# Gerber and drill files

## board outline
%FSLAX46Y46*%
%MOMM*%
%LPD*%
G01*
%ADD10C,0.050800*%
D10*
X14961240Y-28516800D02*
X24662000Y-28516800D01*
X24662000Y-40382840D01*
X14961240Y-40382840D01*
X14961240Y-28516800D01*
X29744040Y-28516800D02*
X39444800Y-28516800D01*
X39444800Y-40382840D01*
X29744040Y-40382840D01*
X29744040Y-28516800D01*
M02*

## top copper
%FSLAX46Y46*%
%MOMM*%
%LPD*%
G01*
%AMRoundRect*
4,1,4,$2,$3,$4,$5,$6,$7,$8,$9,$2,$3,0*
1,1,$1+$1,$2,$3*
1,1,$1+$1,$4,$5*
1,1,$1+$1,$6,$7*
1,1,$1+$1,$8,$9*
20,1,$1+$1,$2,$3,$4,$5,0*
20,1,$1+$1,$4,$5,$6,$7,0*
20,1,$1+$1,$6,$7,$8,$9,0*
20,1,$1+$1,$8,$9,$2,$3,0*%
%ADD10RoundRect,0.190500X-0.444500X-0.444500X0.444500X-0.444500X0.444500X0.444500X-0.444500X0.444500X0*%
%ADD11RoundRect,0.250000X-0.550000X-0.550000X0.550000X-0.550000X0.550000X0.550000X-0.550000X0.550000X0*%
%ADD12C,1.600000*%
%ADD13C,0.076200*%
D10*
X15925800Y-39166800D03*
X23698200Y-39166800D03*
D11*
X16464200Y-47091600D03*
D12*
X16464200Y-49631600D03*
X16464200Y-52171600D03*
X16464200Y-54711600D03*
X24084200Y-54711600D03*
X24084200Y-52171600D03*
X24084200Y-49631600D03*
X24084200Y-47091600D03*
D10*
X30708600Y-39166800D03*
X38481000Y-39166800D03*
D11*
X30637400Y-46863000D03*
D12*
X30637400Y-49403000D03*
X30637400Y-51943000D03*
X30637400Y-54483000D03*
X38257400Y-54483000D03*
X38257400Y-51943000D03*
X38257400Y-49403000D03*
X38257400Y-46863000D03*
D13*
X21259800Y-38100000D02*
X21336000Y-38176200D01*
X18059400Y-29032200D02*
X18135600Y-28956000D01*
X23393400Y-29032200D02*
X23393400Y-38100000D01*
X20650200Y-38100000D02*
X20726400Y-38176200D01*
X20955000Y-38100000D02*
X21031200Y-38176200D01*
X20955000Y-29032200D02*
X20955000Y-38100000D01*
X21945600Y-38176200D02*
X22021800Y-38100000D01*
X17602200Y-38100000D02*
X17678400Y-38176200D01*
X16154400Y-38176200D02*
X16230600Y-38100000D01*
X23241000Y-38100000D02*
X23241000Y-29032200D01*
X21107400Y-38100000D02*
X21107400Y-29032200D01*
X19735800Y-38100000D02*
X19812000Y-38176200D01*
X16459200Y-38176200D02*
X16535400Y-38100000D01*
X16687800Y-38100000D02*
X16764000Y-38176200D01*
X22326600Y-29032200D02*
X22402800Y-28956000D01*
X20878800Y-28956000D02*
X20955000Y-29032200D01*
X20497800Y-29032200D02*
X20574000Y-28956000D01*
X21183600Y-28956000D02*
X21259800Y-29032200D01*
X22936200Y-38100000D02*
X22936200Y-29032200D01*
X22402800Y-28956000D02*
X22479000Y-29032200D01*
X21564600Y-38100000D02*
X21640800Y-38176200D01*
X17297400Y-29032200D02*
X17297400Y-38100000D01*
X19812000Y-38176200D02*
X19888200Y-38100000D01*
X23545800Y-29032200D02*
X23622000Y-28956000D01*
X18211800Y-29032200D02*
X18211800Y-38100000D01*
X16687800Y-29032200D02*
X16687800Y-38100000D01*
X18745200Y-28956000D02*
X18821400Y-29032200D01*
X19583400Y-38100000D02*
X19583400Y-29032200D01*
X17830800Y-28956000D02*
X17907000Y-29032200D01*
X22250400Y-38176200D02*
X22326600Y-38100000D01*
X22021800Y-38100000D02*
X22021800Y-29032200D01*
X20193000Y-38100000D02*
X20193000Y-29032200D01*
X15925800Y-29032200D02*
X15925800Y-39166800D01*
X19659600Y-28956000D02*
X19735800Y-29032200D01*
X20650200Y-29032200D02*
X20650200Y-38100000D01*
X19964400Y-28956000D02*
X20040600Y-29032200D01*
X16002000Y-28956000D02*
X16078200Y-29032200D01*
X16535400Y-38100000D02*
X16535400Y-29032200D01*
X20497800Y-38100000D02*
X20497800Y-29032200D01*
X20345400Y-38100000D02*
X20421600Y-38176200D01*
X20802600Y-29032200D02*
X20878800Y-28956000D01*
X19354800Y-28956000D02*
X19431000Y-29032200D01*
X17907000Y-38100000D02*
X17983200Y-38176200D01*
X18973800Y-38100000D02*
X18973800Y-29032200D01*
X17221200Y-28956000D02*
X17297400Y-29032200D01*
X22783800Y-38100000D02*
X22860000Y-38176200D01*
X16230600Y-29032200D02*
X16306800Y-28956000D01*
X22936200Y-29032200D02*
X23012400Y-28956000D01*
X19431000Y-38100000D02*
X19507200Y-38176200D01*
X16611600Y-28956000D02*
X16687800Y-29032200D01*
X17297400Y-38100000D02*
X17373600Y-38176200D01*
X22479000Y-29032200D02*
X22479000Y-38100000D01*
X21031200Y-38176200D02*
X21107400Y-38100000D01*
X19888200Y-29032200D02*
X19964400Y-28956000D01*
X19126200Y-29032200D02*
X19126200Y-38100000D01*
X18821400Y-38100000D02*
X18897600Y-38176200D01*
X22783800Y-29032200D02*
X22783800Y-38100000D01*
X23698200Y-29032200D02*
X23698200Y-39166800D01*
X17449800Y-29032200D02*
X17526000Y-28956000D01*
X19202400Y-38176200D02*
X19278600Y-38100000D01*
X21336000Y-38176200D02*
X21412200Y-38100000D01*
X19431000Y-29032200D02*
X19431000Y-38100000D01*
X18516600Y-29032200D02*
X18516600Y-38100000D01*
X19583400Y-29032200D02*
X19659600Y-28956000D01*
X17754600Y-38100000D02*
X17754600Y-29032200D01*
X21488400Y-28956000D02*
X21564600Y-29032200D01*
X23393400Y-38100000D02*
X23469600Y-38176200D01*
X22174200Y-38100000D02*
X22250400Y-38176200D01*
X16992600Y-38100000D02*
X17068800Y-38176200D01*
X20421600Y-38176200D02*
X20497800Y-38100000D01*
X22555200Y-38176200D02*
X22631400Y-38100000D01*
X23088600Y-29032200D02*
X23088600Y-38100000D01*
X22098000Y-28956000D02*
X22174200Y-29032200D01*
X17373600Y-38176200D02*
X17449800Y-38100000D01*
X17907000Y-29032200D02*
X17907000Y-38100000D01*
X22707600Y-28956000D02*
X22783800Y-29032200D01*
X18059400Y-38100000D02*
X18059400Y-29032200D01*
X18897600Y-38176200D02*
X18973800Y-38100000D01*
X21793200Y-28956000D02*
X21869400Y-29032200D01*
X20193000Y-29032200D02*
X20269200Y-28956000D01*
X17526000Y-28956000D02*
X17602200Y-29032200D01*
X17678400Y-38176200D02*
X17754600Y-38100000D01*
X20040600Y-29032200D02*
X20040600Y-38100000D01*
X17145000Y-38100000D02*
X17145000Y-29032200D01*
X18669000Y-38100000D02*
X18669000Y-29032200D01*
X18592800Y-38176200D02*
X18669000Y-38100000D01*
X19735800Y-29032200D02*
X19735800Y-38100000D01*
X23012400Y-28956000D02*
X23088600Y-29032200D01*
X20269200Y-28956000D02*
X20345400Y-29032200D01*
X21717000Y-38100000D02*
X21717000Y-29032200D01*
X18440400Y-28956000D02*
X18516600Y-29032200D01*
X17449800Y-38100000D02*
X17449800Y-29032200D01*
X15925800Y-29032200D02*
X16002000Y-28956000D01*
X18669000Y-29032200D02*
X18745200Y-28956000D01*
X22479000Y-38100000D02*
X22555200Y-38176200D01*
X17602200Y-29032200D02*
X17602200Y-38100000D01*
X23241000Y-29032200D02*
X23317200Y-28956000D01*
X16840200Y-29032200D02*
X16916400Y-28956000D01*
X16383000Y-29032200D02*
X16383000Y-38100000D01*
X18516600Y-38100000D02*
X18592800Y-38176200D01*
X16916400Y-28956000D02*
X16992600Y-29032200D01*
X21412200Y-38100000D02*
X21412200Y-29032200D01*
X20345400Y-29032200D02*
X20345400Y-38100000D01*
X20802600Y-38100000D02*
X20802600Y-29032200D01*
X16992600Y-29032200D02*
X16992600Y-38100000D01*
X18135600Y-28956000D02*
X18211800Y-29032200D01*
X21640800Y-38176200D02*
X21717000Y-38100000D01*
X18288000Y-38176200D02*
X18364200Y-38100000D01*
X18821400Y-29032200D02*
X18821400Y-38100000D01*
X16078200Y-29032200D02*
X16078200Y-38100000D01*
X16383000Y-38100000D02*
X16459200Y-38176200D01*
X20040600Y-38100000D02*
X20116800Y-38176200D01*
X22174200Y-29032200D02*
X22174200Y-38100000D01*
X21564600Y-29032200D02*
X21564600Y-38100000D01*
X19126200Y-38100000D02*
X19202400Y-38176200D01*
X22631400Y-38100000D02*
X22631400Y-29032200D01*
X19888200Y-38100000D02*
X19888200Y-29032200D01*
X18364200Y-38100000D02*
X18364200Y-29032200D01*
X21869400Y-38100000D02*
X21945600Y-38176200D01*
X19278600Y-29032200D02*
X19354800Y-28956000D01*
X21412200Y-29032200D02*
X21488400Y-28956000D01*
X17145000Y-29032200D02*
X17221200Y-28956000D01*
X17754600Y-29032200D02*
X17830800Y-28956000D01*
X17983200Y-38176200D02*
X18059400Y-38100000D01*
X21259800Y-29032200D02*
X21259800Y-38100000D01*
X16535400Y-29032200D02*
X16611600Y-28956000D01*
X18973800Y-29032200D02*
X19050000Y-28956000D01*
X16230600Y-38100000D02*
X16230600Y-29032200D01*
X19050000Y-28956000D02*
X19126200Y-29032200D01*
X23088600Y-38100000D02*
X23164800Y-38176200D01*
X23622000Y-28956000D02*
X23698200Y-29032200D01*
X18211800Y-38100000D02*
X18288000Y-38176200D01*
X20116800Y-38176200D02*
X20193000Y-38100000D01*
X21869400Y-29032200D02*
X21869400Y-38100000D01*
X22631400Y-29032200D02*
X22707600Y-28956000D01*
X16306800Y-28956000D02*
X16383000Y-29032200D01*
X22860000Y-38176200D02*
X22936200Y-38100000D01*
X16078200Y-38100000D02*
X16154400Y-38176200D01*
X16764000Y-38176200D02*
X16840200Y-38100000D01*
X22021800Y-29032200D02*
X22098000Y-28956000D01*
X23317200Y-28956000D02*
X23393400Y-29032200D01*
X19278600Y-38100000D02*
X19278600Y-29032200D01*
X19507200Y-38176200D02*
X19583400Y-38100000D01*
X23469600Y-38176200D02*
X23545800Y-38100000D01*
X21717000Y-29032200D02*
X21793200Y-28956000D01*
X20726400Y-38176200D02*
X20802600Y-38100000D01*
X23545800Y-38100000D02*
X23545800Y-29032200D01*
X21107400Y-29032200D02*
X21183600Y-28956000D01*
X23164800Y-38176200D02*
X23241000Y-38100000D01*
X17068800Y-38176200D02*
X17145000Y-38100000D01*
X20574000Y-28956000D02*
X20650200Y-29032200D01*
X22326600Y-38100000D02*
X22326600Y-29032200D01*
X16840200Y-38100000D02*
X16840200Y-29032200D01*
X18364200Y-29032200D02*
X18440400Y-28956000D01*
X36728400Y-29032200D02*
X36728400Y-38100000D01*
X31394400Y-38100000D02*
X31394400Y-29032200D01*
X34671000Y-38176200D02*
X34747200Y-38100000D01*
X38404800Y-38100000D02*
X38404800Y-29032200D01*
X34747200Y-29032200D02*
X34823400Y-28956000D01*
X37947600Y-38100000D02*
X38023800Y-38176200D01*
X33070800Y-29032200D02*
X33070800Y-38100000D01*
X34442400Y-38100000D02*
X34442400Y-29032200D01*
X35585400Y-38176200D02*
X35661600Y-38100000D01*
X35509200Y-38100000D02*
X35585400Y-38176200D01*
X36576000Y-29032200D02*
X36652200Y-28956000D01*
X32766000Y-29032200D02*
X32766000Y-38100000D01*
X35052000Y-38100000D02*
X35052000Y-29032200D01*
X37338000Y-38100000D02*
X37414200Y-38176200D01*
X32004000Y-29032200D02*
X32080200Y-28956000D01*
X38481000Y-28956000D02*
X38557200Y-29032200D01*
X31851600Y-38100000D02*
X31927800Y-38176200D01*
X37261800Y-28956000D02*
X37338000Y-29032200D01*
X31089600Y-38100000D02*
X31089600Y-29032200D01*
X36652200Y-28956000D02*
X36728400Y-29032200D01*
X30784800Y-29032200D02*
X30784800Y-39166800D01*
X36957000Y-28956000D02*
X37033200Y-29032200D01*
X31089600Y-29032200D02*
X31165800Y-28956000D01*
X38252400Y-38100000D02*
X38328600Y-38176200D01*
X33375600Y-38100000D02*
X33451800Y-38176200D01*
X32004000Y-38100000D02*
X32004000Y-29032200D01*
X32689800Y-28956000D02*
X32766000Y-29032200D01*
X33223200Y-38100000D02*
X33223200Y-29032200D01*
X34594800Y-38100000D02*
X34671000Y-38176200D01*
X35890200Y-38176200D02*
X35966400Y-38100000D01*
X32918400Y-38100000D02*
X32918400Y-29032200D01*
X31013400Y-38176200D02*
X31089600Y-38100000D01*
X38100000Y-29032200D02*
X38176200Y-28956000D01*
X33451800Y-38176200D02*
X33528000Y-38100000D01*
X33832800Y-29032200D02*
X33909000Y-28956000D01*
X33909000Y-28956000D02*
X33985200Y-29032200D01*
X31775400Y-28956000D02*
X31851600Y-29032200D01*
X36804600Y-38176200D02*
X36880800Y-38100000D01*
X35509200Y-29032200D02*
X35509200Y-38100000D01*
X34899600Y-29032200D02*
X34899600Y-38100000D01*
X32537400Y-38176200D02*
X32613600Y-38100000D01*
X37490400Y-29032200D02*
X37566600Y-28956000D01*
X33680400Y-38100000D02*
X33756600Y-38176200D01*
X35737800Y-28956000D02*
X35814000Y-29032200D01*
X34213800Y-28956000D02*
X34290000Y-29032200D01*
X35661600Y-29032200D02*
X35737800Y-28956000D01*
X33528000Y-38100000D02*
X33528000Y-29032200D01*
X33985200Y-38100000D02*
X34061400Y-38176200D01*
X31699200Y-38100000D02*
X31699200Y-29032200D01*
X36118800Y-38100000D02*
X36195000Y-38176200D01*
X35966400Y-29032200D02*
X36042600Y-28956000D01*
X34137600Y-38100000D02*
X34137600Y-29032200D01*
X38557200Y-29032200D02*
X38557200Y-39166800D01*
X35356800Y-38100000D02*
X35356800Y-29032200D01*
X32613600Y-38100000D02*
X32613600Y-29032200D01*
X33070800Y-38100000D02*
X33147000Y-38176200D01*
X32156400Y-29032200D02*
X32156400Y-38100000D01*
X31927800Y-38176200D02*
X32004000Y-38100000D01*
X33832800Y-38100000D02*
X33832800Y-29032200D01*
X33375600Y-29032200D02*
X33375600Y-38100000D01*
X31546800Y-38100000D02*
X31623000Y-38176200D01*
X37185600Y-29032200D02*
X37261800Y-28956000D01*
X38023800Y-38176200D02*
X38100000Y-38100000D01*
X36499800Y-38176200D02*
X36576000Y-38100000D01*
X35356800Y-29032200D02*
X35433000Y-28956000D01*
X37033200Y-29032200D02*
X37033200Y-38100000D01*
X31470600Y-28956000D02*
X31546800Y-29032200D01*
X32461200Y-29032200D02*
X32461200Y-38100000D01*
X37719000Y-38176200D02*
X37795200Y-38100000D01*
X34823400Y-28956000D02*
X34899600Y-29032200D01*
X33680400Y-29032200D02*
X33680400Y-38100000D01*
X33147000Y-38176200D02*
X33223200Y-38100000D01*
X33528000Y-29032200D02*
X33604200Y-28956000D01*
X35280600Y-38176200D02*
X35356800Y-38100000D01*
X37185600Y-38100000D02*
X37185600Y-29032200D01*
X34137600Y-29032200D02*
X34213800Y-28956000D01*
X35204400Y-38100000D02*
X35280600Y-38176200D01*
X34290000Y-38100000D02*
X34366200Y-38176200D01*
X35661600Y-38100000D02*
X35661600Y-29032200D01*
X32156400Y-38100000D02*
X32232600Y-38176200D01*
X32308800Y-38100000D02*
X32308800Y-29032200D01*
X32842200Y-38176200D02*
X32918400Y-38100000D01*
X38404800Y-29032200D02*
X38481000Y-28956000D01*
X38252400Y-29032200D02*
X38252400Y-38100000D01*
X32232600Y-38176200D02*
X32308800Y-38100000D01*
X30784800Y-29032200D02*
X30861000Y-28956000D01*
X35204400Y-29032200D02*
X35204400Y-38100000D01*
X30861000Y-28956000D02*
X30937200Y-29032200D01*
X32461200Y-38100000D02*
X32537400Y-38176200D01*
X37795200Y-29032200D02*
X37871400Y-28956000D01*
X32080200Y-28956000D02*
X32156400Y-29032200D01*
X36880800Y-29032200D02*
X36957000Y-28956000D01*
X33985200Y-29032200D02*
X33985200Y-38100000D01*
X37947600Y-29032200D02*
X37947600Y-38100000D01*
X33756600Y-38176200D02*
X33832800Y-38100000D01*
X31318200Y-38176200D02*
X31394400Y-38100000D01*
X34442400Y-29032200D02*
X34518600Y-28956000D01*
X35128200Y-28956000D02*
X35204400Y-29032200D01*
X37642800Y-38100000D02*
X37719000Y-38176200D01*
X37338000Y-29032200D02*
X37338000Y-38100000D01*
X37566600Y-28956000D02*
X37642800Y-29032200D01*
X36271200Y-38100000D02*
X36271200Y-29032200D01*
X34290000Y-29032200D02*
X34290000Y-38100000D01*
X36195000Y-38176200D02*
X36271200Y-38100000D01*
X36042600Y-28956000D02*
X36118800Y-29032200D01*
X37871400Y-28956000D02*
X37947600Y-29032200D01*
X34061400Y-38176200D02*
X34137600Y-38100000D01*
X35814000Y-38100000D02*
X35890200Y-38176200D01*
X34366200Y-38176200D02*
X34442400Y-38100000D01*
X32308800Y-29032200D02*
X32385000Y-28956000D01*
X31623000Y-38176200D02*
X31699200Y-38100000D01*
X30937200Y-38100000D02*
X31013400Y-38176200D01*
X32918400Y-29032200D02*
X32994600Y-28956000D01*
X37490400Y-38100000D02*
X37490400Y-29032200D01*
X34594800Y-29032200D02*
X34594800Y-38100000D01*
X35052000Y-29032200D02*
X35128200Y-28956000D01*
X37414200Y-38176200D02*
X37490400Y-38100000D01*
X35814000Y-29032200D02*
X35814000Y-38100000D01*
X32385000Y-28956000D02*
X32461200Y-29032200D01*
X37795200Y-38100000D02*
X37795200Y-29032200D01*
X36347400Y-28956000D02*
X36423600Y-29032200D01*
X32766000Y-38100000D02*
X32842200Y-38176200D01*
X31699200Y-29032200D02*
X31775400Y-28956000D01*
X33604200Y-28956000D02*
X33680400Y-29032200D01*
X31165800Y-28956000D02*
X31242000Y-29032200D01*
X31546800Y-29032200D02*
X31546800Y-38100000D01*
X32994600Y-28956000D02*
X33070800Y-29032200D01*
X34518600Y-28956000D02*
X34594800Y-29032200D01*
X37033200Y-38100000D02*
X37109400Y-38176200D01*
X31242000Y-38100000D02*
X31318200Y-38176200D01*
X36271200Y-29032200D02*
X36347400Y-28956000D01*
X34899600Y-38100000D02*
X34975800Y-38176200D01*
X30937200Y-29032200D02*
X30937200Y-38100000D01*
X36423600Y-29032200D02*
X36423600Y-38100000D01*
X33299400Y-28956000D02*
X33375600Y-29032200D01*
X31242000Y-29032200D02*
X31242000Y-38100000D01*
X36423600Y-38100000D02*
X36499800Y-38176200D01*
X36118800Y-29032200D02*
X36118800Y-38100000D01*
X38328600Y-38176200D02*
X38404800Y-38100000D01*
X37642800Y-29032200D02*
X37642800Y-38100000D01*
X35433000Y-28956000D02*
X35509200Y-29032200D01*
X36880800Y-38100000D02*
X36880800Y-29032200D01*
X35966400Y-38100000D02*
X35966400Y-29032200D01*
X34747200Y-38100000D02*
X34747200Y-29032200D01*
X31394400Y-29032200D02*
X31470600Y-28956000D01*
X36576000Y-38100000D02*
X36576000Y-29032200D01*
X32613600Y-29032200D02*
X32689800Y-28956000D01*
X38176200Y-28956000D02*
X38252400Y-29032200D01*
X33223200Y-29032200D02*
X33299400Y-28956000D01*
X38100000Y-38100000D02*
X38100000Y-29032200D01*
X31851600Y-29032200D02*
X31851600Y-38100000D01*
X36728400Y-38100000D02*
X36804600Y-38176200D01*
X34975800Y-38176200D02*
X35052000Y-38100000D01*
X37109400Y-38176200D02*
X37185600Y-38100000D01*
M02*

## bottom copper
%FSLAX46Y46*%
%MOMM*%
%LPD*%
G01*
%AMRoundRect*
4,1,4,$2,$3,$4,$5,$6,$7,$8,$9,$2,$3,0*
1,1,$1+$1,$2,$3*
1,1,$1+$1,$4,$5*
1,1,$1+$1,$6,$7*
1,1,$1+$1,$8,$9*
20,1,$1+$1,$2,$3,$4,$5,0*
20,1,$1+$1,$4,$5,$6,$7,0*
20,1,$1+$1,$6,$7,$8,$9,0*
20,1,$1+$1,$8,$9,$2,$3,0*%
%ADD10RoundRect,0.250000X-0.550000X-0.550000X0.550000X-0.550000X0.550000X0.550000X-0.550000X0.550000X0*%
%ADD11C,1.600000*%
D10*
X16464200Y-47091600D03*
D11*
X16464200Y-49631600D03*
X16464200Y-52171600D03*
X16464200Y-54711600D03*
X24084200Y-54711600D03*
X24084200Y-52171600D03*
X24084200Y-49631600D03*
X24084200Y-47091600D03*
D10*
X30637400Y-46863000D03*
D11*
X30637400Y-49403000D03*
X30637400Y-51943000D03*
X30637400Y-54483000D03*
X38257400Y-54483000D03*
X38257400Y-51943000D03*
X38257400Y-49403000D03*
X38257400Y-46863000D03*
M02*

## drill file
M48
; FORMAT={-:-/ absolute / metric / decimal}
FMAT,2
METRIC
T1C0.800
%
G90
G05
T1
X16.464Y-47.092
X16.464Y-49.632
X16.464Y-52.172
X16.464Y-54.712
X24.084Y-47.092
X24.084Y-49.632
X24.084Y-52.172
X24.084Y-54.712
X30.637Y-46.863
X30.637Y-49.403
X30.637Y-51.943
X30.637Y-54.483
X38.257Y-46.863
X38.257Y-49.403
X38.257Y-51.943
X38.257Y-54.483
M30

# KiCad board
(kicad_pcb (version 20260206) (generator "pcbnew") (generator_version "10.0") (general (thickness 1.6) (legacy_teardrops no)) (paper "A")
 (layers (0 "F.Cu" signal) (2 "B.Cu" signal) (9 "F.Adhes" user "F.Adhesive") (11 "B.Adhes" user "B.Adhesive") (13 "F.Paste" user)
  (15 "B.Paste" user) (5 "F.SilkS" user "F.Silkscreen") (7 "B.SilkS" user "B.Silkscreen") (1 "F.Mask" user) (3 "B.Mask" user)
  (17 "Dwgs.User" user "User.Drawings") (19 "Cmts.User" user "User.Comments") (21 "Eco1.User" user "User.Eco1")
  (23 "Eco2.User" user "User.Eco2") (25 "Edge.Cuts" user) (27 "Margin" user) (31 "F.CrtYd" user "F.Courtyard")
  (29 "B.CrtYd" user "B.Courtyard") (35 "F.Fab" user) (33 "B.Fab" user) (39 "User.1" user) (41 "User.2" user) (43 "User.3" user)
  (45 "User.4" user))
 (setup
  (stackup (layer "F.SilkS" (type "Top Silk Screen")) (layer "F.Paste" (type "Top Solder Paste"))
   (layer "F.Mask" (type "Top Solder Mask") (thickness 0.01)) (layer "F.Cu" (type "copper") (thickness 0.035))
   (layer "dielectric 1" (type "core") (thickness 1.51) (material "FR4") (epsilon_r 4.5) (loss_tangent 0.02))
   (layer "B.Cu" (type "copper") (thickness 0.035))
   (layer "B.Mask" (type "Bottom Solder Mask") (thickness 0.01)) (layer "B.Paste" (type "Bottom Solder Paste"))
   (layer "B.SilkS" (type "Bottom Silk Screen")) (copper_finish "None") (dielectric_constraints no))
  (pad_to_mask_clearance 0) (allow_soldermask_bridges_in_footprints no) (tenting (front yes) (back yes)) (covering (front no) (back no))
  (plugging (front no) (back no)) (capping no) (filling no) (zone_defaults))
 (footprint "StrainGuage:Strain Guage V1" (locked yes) (layer "F.Cu") (at 19.812 39.1668)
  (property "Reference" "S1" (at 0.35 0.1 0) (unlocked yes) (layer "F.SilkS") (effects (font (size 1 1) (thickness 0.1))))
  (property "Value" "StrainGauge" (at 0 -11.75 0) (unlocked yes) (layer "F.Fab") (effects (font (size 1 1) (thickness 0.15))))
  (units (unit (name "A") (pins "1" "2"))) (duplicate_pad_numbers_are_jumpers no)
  (fp_rect (start -4.85076 -10.65) (end 4.85 1.21604) (stroke (width 0.0508) (type solid)) (fill no) (layer "Edge.Cuts"))
  (pad "1" smd roundrect (at -3.8862 0) (size 1.27 1.27) (layers "F.Cu" "F.Mask" "F.Paste") (roundrect_rratio 0.15) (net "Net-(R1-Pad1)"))
  (pad "2" smd roundrect (at 3.8862 0) (size 1.27 1.27) (layers "F.Cu" "F.Mask" "F.Paste") (roundrect_rratio 0.15) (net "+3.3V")))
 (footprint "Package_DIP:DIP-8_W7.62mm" (layer "F.Cu") (at 16.4642 47.0916)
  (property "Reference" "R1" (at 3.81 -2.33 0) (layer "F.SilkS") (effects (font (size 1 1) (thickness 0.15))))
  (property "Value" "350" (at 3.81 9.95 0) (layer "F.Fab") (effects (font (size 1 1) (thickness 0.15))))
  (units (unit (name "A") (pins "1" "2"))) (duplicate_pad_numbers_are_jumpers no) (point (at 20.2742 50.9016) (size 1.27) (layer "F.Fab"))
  (pad "1" thru_hole roundrect (at 0 0) (size 1.6 1.6) (drill 0.8) (layers "*.Cu" "*.Mask") (remove_unused_layers no)
   (roundrect_rratio 0.15625) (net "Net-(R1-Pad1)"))
  (pad "2" thru_hole circle (at 0 2.54) (size 1.6 1.6) (drill 0.8) (layers "*.Cu" "*.Mask") (remove_unused_layers no) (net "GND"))
  (pad "3" thru_hole circle (at 0 5.08) (size 1.6 1.6) (drill 0.8) (layers "*.Cu" "*.Mask") (remove_unused_layers no))
  (pad "4" thru_hole circle (at 0 7.62) (size 1.6 1.6) (drill 0.8) (layers "*.Cu" "*.Mask") (remove_unused_layers no))
  (pad "5" thru_hole circle (at 7.62 7.62) (size 1.6 1.6) (drill 0.8) (layers "*.Cu" "*.Mask") (remove_unused_layers no))
  (pad "6" thru_hole circle (at 7.62 5.08) (size 1.6 1.6) (drill 0.8) (layers "*.Cu" "*.Mask") (remove_unused_layers no))
  (pad "7" thru_hole circle (at 7.62 2.54) (size 1.6 1.6) (drill 0.8) (layers "*.Cu" "*.Mask") (remove_unused_layers no))
  (pad "8" thru_hole circle (at 7.62 0) (size 1.6 1.6) (drill 0.8) (layers "*.Cu" "*.Mask") (remove_unused_layers no)))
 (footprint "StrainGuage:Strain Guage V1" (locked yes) (layer "F.Cu") (at 34.5948 39.1668)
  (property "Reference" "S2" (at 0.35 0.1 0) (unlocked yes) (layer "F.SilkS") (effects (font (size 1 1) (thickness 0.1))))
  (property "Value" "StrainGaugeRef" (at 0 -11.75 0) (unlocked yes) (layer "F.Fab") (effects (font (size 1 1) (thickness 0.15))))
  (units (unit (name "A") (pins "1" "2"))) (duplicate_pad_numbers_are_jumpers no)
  (fp_rect (start -4.85076 -10.65) (end 4.85 1.21604) (stroke (width 0.0508) (type solid)) (fill no) (layer "Edge.Cuts"))
  (pad "1" smd roundrect (at -3.8862 0) (size 1.27 1.27) (layers "F.Cu" "F.Mask" "F.Paste") (roundrect_rratio 0.15) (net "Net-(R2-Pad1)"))
  (pad "2" smd roundrect (at 3.8862 0) (size 1.27 1.27) (layers "F.Cu" "F.Mask" "F.Paste") (roundrect_rratio 0.15) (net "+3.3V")))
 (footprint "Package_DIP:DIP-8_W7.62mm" (layer "F.Cu") (at 30.6374 46.863)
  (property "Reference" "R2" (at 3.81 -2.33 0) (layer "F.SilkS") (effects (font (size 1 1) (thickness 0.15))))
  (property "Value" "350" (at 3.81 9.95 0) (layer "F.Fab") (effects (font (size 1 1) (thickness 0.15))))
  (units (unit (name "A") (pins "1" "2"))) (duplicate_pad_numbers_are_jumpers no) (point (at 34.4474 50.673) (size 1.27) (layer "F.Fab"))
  (pad "1" thru_hole roundrect (at 0 0) (size 1.6 1.6) (drill 0.8) (layers "*.Cu" "*.Mask") (remove_unused_layers no)
   (roundrect_rratio 0.15625) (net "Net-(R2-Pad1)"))
  (pad "2" thru_hole circle (at 0 2.54) (size 1.6 1.6) (drill 0.8) (layers "*.Cu" "*.Mask") (remove_unused_layers no) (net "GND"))
  (pad "3" thru_hole circle (at 0 5.08) (size 1.6 1.6) (drill 0.8) (layers "*.Cu" "*.Mask") (remove_unused_layers no))
  (pad "4" thru_hole circle (at 0 7.62) (size 1.6 1.6) (drill 0.8) (layers "*.Cu" "*.Mask") (remove_unused_layers no))
  (pad "5" thru_hole circle (at 7.62 7.62) (size 1.6 1.6) (drill 0.8) (layers "*.Cu" "*.Mask") (remove_unused_layers no))
  (pad "6" thru_hole circle (at 7.62 5.08) (size 1.6 1.6) (drill 0.8) (layers "*.Cu" "*.Mask") (remove_unused_layers no))
  (pad "7" thru_hole circle (at 7.62 2.54) (size 1.6 1.6) (drill 0.8) (layers "*.Cu" "*.Mask") (remove_unused_layers no))
  (pad "8" thru_hole circle (at 7.62 0) (size 1.6 1.6) (drill 0.8) (layers "*.Cu" "*.Mask") (remove_unused_layers no)))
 (segment (start 21.2598 38.1) (end 21.336 38.1762) (width 0.0762) (layer "F.Cu") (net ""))
 (segment (start 18.0594 29.0322) (end 18.1356 28.956) (width 0.0762) (layer "F.Cu") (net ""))
 (segment (start 23.3934 29.0322) (end 23.3934 38.1) (width 0.0762) (layer "F.Cu") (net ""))
 (segment (start 20.6502 38.1) (end 20.7264 38.1762) (width 0.0762) (layer "F.Cu") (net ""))
 (segment (start 20.955 38.1) (end 21.0312 38.1762) (width 0.0762) (layer "F.Cu") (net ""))
 (segment (start 20.955 29.0322) (end 20.955 38.1) (width 0.0762) (layer "F.Cu") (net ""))
 (segment (start 21.9456 38.1762) (end 22.0218 38.1) (width 0.0762) (layer "F.Cu") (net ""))
 (segment (start 17.6022 38.1) (end 17.6784 38.1762) (width 0.0762) (layer "F.Cu") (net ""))
 (segment (start 16.1544 38.1762) (end 16.2306 38.1) (width 0.0762) (layer "F.Cu") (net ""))
 (segment (start 23.241 38.1) (end 23.241 29.0322) (width 0.0762) (layer "F.Cu") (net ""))
 (segment (start 21.1074 38.1) (end 21.1074 29.0322) (width 0.0762) (layer "F.Cu") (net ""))
 (segment (start 19.7358 38.1) (end 19.812 38.1762) (width 0.0762) (layer "F.Cu") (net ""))
 (segment (start 16.4592 38.1762) (end 16.5354 38.1) (width 0.0762) (layer "F.Cu") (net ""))
 (segment (start 16.6878 38.1) (end 16.764 38.1762) (width 0.0762) (layer "F.Cu") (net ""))
 (segment (start 22.3266 29.0322) (end 22.4028 28.956) (width 0.0762) (layer "F.Cu") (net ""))
 (segment (start 20.8788 28.956) (end 20.955 29.0322) (width 0.0762) (layer "F.Cu") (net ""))
 (segment (start 20.4978 29.0322) (end 20.574 28.956) (width 0.0762) (layer "F.Cu") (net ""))
 (segment (start 21.1836 28.956) (end 21.2598 29.0322) (width 0.0762) (layer "F.Cu") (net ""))
 (segment (start 22.9362 38.1) (end 22.9362 29.0322) (width 0.0762) (layer "F.Cu") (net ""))
 (segment (start 22.4028 28.956) (end 22.479 29.0322) (width 0.0762) (layer "F.Cu") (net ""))
 (segment (start 21.5646 38.1) (end 21.6408 38.1762) (width 0.0762) (layer "F.Cu") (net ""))
 (segment (start 17.2974 29.0322) (end 17.2974 38.1) (width 0.0762) (layer "F.Cu") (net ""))
 (segment (start 19.812 38.1762) (end 19.8882 38.1) (width 0.0762) (layer "F.Cu") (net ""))
 (segment (start 23.5458 29.0322) (end 23.622 28.956) (width 0.0762) (layer "F.Cu") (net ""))
 (segment (start 18.2118 29.0322) (end 18.2118 38.1) (width 0.0762) (layer "F.Cu") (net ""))
 (segment (start 16.6878 29.0322) (end 16.6878 38.1) (width 0.0762) (layer "F.Cu") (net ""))
 (segment (start 18.7452 28.956) (end 18.8214 29.0322) (width 0.0762) (layer "F.Cu") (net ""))
 (segment (start 19.5834 38.1) (end 19.5834 29.0322) (width 0.0762) (layer "F.Cu") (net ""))
 (segment (start 17.8308 28.956) (end 17.907 29.0322) (width 0.0762) (layer "F.Cu") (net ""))
 (segment (start 22.2504 38.1762) (end 22.3266 38.1) (width 0.0762) (layer "F.Cu") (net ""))
 (segment (start 22.0218 38.1) (end 22.0218 29.0322) (width 0.0762) (layer "F.Cu") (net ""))
 (segment (start 20.193 38.1) (end 20.193 29.0322) (width 0.0762) (layer "F.Cu") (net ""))
 (segment (start 15.9258 29.0322) (end 15.9258 39.1668) (width 0.0762) (layer "F.Cu") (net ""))
 (segment (start 19.6596 28.956) (end 19.7358 29.0322) (width 0.0762) (layer "F.Cu") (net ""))
 (segment (start 20.6502 29.0322) (end 20.6502 38.1) (width 0.0762) (layer "F.Cu") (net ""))
 (segment (start 19.9644 28.956) (end 20.0406 29.0322) (width 0.0762) (layer "F.Cu") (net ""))
 (segment (start 16.002 28.956) (end 16.0782 29.0322) (width 0.0762) (layer "F.Cu") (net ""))
 (segment (start 16.5354 38.1) (end 16.5354 29.0322) (width 0.0762) (layer "F.Cu") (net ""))
 (segment (start 20.4978 38.1) (end 20.4978 29.0322) (width 0.0762) (layer "F.Cu") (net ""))
 (segment (start 20.3454 38.1) (end 20.4216 38.1762) (width 0.0762) (layer "F.Cu") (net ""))
 (segment (start 20.8026 29.0322) (end 20.8788 28.956) (width 0.0762) (layer "F.Cu") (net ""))
 (segment (start 19.3548 28.956) (end 19.431 29.0322) (width 0.0762) (layer "F.Cu") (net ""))
 (segment (start 17.907 38.1) (end 17.9832 38.1762) (width 0.0762) (layer "F.Cu") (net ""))
 (segment (start 18.9738 38.1) (end 18.9738 29.0322) (width 0.0762) (layer "F.Cu") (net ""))
 (segment (start 17.2212 28.956) (end 17.2974 29.0322) (width 0.0762) (layer "F.Cu") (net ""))
 (segment (start 22.7838 38.1) (end 22.86 38.1762) (width 0.0762) (layer "F.Cu") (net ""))
 (segment (start 16.2306 29.0322) (end 16.3068 28.956) (width 0.0762) (layer "F.Cu") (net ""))
 (segment (start 22.9362 29.0322) (end 23.0124 28.956) (width 0.0762) (layer "F.Cu") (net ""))
 (segment (start 19.431 38.1) (end 19.5072 38.1762) (width 0.0762) (layer "F.Cu") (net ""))
 (segment (start 16.6116 28.956) (end 16.6878 29.0322) (width 0.0762) (layer "F.Cu") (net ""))
 (segment (start 17.2974 38.1) (end 17.3736 38.1762) (width 0.0762) (layer "F.Cu") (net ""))
 (segment (start 22.479 29.0322) (end 22.479 38.1) (width 0.0762) (layer "F.Cu") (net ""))
 (segment (start 21.0312 38.1762) (end 21.1074 38.1) (width 0.0762) (layer "F.Cu") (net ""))
 (segment (start 19.8882 29.0322) (end 19.9644 28.956) (width 0.0762) (layer "F.Cu") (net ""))
 (segment (start 19.1262 29.0322) (end 19.1262 38.1) (width 0.0762) (layer "F.Cu") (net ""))
 (segment (start 18.8214 38.1) (end 18.8976 38.1762) (width 0.0762) (layer "F.Cu") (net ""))
 (segment (start 22.7838 29.0322) (end 22.7838 38.1) (width 0.0762) (layer "F.Cu") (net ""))
 (segment (start 23.6982 29.0322) (end 23.6982 39.1668) (width 0.0762) (layer "F.Cu") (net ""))
 (segment (start 17.4498 29.0322) (end 17.526 28.956) (width 0.0762) (layer "F.Cu") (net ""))
 (segment (start 19.2024 38.1762) (end 19.2786 38.1) (width 0.0762) (layer "F.Cu") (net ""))
 (segment (start 21.336 38.1762) (end 21.4122 38.1) (width 0.0762) (layer "F.Cu") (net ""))
 (segment (start 19.431 29.0322) (end 19.431 38.1) (width 0.0762) (layer "F.Cu") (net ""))
 (segment (start 18.5166 29.0322) (end 18.5166 38.1) (width 0.0762) (layer "F.Cu") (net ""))
 (segment (start 19.5834 29.0322) (end 19.6596 28.956) (width 0.0762) (layer "F.Cu") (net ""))
 (segment (start 17.7546 38.1) (end 17.7546 29.0322) (width 0.0762) (layer "F.Cu") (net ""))
 (segment (start 21.4884 28.956) (end 21.5646 29.0322) (width 0.0762) (layer "F.Cu") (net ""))
 (segment (start 23.3934 38.1) (end 23.4696 38.1762) (width 0.0762) (layer "F.Cu") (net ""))
 (segment (start 22.1742 38.1) (end 22.2504 38.1762) (width 0.0762) (layer "F.Cu") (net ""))
 (segment (start 16.9926 38.1) (end 17.0688 38.1762) (width 0.0762) (layer "F.Cu") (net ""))
 (segment (start 20.4216 38.1762) (end 20.4978 38.1) (width 0.0762) (layer "F.Cu") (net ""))
 (segment (start 22.5552 38.1762) (end 22.6314 38.1) (width 0.0762) (layer "F.Cu") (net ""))
 (segment (start 23.0886 29.0322) (end 23.0886 38.1) (width 0.0762) (layer "F.Cu") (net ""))
 (segment (start 22.098 28.956) (end 22.1742 29.0322) (width 0.0762) (layer "F.Cu") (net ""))
 (segment (start 17.3736 38.1762) (end 17.4498 38.1) (width 0.0762) (layer "F.Cu") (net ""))
 (segment (start 17.907 29.0322) (end 17.907 38.1) (width 0.0762) (layer "F.Cu") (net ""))
 (segment (start 22.7076 28.956) (end 22.7838 29.0322) (width 0.0762) (layer "F.Cu") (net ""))
 (segment (start 18.0594 38.1) (end 18.0594 29.0322) (width 0.0762) (layer "F.Cu") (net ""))
 (segment (start 18.8976 38.1762) (end 18.9738 38.1) (width 0.0762) (layer "F.Cu") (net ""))
 (segment (start 21.7932 28.956) (end 21.8694 29.0322) (width 0.0762) (layer "F.Cu") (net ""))
 (segment (start 20.193 29.0322) (end 20.2692 28.956) (width 0.0762) (layer "F.Cu") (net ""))
 (segment (start 17.526 28.956) (end 17.6022 29.0322) (width 0.0762) (layer "F.Cu") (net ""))
 (segment (start 17.6784 38.1762) (end 17.7546 38.1) (width 0.0762) (layer "F.Cu") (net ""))
 (segment (start 20.0406 29.0322) (end 20.0406 38.1) (width 0.0762) (layer "F.Cu") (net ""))
 (segment (start 17.145 38.1) (end 17.145 29.0322) (width 0.0762) (layer "F.Cu") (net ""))
 (segment (start 18.669 38.1) (end 18.669 29.0322) (width 0.0762) (layer "F.Cu") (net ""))
 (segment (start 18.5928 38.1762) (end 18.669 38.1) (width 0.0762) (layer "F.Cu") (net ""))
 (segment (start 19.7358 29.0322) (end 19.7358 38.1) (width 0.0762) (layer "F.Cu") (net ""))
 (segment (start 23.0124 28.956) (end 23.0886 29.0322) (width 0.0762) (layer "F.Cu") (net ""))
 (segment (start 20.2692 28.956) (end 20.3454 29.0322) (width 0.0762) (layer "F.Cu") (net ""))
 (segment (start 21.717 38.1) (end 21.717 29.0322) (width 0.0762) (layer "F.Cu") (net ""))
 (segment (start 18.4404 28.956) (end 18.5166 29.0322) (width 0.0762) (layer "F.Cu") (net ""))
 (segment (start 17.4498 38.1) (end 17.4498 29.0322) (width 0.0762) (layer "F.Cu") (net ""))
 (segment (start 15.9258 29.0322) (end 16.002 28.956) (width 0.0762) (layer "F.Cu") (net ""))
 (segment (start 18.669 29.0322) (end 18.7452 28.956) (width 0.0762) (layer "F.Cu") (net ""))
 (segment (start 22.479 38.1) (end 22.5552 38.1762) (width 0.0762) (layer "F.Cu") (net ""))
 (segment (start 17.6022 29.0322) (end 17.6022 38.1) (width 0.0762) (layer "F.Cu") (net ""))
 (segment (start 23.241 29.0322) (end 23.3172 28.956) (width 0.0762) (layer "F.Cu") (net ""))
 (segment (start 16.8402 29.0322) (end 16.9164 28.956) (width 0.0762) (layer "F.Cu") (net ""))
 (segment (start 16.383 29.0322) (end 16.383 38.1) (width 0.0762) (layer "F.Cu") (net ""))
 (segment (start 18.5166 38.1) (end 18.5928 38.1762) (width 0.0762) (layer "F.Cu") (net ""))
 (segment (start 16.9164 28.956) (end 16.9926 29.0322) (width 0.0762) (layer "F.Cu") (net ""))
 (segment (start 21.4122 38.1) (end 21.4122 29.0322) (width 0.0762) (layer "F.Cu") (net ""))
 (segment (start 20.3454 29.0322) (end 20.3454 38.1) (width 0.0762) (layer "F.Cu") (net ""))
 (segment (start 20.8026 38.1) (end 20.8026 29.0322) (width 0.0762) (layer "F.Cu") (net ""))
 (segment (start 16.9926 29.0322) (end 16.9926 38.1) (width 0.0762) (layer "F.Cu") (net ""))
 (segment (start 18.1356 28.956) (end 18.2118 29.0322) (width 0.0762) (layer "F.Cu") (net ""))
 (segment (start 21.6408 38.1762) (end 21.717 38.1) (width 0.0762) (layer "F.Cu") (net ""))
 (segment (start 18.288 38.1762) (end 18.3642 38.1) (width 0.0762) (layer "F.Cu") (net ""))
 (segment (start 18.8214 29.0322) (end 18.8214 38.1) (width 0.0762) (layer "F.Cu") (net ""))
 (segment (start 16.0782 29.0322) (end 16.0782 38.1) (width 0.0762) (layer "F.Cu") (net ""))
 (segment (start 16.383 38.1) (end 16.4592 38.1762) (width 0.0762) (layer "F.Cu") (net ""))
 (segment (start 20.0406 38.1) (end 20.1168 38.1762) (width 0.0762) (layer "F.Cu") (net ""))
 (segment (start 22.1742 29.0322) (end 22.1742 38.1) (width 0.0762) (layer "F.Cu") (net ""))
 (segment (start 21.5646 29.0322) (end 21.5646 38.1) (width 0.0762) (layer "F.Cu") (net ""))
 (segment (start 19.1262 38.1) (end 19.2024 38.1762) (width 0.0762) (layer "F.Cu") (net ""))
 (segment (start 22.6314 38.1) (end 22.6314 29.0322) (width 0.0762) (layer "F.Cu") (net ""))
 (segment (start 19.8882 38.1) (end 19.8882 29.0322) (width 0.0762) (layer "F.Cu") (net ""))
 (segment (start 18.3642 38.1) (end 18.3642 29.0322) (width 0.0762) (layer "F.Cu") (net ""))
 (segment (start 21.8694 38.1) (end 21.9456 38.1762) (width 0.0762) (layer "F.Cu") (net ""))
 (segment (start 19.2786 29.0322) (end 19.3548 28.956) (width 0.0762) (layer "F.Cu") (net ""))
 (segment (start 21.4122 29.0322) (end 21.4884 28.956) (width 0.0762) (layer "F.Cu") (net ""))
 (segment (start 17.145 29.0322) (end 17.2212 28.956) (width 0.0762) (layer "F.Cu") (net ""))
 (segment (start 17.7546 29.0322) (end 17.8308 28.956) (width 0.0762) (layer "F.Cu") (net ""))
 (segment (start 17.9832 38.1762) (end 18.0594 38.1) (width 0.0762) (layer "F.Cu") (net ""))
 (segment (start 21.2598 29.0322) (end 21.2598 38.1) (width 0.0762) (layer "F.Cu") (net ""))
 (segment (start 16.5354 29.0322) (end 16.6116 28.956) (width 0.0762) (layer "F.Cu") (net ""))
 (segment (start 18.9738 29.0322) (end 19.05 28.956) (width 0.0762) (layer "F.Cu") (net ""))
 (segment (start 16.2306 38.1) (end 16.2306 29.0322) (width 0.0762) (layer "F.Cu") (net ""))
 (segment (start 19.05 28.956) (end 19.1262 29.0322) (width 0.0762) (layer "F.Cu") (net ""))
 (segment (start 23.0886 38.1) (end 23.1648 38.1762) (width 0.0762) (layer "F.Cu") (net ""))
 (segment (start 23.622 28.956) (end 23.6982 29.0322) (width 0.0762) (layer "F.Cu") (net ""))
 (segment (start 18.2118 38.1) (end 18.288 38.1762) (width 0.0762) (layer "F.Cu") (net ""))
 (segment (start 20.1168 38.1762) (end 20.193 38.1) (width 0.0762) (layer "F.Cu") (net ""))
 (segment (start 21.8694 29.0322) (end 21.8694 38.1) (width 0.0762) (layer "F.Cu") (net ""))
 (segment (start 22.6314 29.0322) (end 22.7076 28.956) (width 0.0762) (layer "F.Cu") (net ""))
 (segment (start 16.3068 28.956) (end 16.383 29.0322) (width 0.0762) (layer "F.Cu") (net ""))
 (segment (start 22.86 38.1762) (end 22.9362 38.1) (width 0.0762) (layer "F.Cu") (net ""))
 (segment (start 16.0782 38.1) (end 16.1544 38.1762) (width 0.0762) (layer "F.Cu") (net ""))
 (segment (start 16.764 38.1762) (end 16.8402 38.1) (width 0.0762) (layer "F.Cu") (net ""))
 (segment (start 22.0218 29.0322) (end 22.098 28.956) (width 0.0762) (layer "F.Cu") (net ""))
 (segment (start 23.3172 28.956) (end 23.3934 29.0322) (width 0.0762) (layer "F.Cu") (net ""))
 (segment (start 19.2786 38.1) (end 19.2786 29.0322) (width 0.0762) (layer "F.Cu") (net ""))
 (segment (start 19.5072 38.1762) (end 19.5834 38.1) (width 0.0762) (layer "F.Cu") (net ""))
 (segment (start 23.4696 38.1762) (end 23.5458 38.1) (width 0.0762) (layer "F.Cu") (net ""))
 (segment (start 21.717 29.0322) (end 21.7932 28.956) (width 0.0762) (layer "F.Cu") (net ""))
 (segment (start 20.7264 38.1762) (end 20.8026 38.1) (width 0.0762) (layer "F.Cu") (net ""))
 (segment (start 23.5458 38.1) (end 23.5458 29.0322) (width 0.0762) (layer "F.Cu") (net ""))
 (segment (start 21.1074 29.0322) (end 21.1836 28.956) (width 0.0762) (layer "F.Cu") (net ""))
 (segment (start 23.1648 38.1762) (end 23.241 38.1) (width 0.0762) (layer "F.Cu") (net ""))
 (segment (start 17.0688 38.1762) (end 17.145 38.1) (width 0.0762) (layer "F.Cu") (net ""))
 (segment (start 20.574 28.956) (end 20.6502 29.0322) (width 0.0762) (layer "F.Cu") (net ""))
 (segment (start 22.3266 38.1) (end 22.3266 29.0322) (width 0.0762) (layer "F.Cu") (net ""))
 (segment (start 16.8402 38.1) (end 16.8402 29.0322) (width 0.0762) (layer "F.Cu") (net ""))
 (segment (start 18.3642 29.0322) (end 18.4404 28.956) (width 0.0762) (layer "F.Cu") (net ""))
 (segment (start 36.7284 29.0322) (end 36.7284 38.1) (width 0.0762) (layer "F.Cu") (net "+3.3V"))
 (segment (start 31.3944 38.1) (end 31.3944 29.0322) (width 0.0762) (layer "F.Cu") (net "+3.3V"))
 (segment (start 34.671 38.1762) (end 34.7472 38.1) (width 0.0762) (layer "F.Cu") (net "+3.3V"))
 (segment (start 38.4048 38.1) (end 38.4048 29.0322) (width 0.0762) (layer "F.Cu") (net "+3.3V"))
 (segment (start 34.7472 29.0322) (end 34.8234 28.956) (width 0.0762) (layer "F.Cu") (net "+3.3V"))
 (segment (start 37.9476 38.1) (end 38.0238 38.1762) (width 0.0762) (layer "F.Cu") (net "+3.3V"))
 (segment (start 33.0708 29.0322) (end 33.0708 38.1) (width 0.0762) (layer "F.Cu") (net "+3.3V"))
 (segment (start 34.4424 38.1) (end 34.4424 29.0322) (width 0.0762) (layer "F.Cu") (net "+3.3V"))
 (segment (start 35.5854 38.1762) (end 35.6616 38.1) (width 0.0762) (layer "F.Cu") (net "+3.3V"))
 (segment (start 35.5092 38.1) (end 35.5854 38.1762) (width 0.0762) (layer "F.Cu") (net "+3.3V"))
 (segment (start 36.576 29.0322) (end 36.6522 28.956) (width 0.0762) (layer "F.Cu") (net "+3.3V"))
 (segment (start 32.766 29.0322) (end 32.766 38.1) (width 0.0762) (layer "F.Cu") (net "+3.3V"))
 (segment (start 35.052 38.1) (end 35.052 29.0322) (width 0.0762) (layer "F.Cu") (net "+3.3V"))
 (segment (start 37.338 38.1) (end 37.4142 38.1762) (width 0.0762) (layer "F.Cu") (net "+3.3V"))
 (segment (start 32.004 29.0322) (end 32.0802 28.956) (width 0.0762) (layer "F.Cu") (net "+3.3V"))
 (segment (start 38.481 28.956) (end 38.5572 29.0322) (width 0.0762) (layer "F.Cu") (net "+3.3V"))
 (segment (start 31.8516 38.1) (end 31.9278 38.1762) (width 0.0762) (layer "F.Cu") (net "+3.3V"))
 (segment (start 37.2618 28.956) (end 37.338 29.0322) (width 0.0762) (layer "F.Cu") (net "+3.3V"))
 (segment (start 31.0896 38.1) (end 31.0896 29.0322) (width 0.0762) (layer "F.Cu") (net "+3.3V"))
 (segment (start 36.6522 28.956) (end 36.7284 29.0322) (width 0.0762) (layer "F.Cu") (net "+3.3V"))
 (segment (start 30.7848 29.0322) (end 30.7848 39.1668) (width 0.0762) (layer "F.Cu") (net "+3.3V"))
 (segment (start 36.957 28.956) (end 37.0332 29.0322) (width 0.0762) (layer "F.Cu") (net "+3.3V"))
 (segment (start 31.0896 29.0322) (end 31.1658 28.956) (width 0.0762) (layer "F.Cu") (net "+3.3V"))
 (segment (start 38.2524 38.1) (end 38.3286 38.1762) (width 0.0762) (layer "F.Cu") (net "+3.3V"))
 (segment (start 33.3756 38.1) (end 33.4518 38.1762) (width 0.0762) (layer "F.Cu") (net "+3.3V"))
 (segment (start 32.004 38.1) (end 32.004 29.0322) (width 0.0762) (layer "F.Cu") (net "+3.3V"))
 (segment (start 32.6898 28.956) (end 32.766 29.0322) (width 0.0762) (layer "F.Cu") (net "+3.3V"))
 (segment (start 33.2232 38.1) (end 33.2232 29.0322) (width 0.0762) (layer "F.Cu") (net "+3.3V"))
 (segment (start 34.5948 38.1) (end 34.671 38.1762) (width 0.0762) (layer "F.Cu") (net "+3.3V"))
 (segment (start 35.8902 38.1762) (end 35.9664 38.1) (width 0.0762) (layer "F.Cu") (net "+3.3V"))
 (segment (start 32.9184 38.1) (end 32.9184 29.0322) (width 0.0762) (layer "F.Cu") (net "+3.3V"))
 (segment (start 31.0134 38.1762) (end 31.0896 38.1) (width 0.0762) (layer "F.Cu") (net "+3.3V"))
 (segment (start 38.1 29.0322) (end 38.1762 28.956) (width 0.0762) (layer "F.Cu") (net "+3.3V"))
 (segment (start 33.4518 38.1762) (end 33.528 38.1) (width 0.0762) (layer "F.Cu") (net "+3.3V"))
 (segment (start 33.8328 29.0322) (end 33.909 28.956) (width 0.0762) (layer "F.Cu") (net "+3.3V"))
 (segment (start 33.909 28.956) (end 33.9852 29.0322) (width 0.0762) (layer "F.Cu") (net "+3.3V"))
 (segment (start 31.7754 28.956) (end 31.8516 29.0322) (width 0.0762) (layer "F.Cu") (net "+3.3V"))
 (segment (start 36.8046 38.1762) (end 36.8808 38.1) (width 0.0762) (layer "F.Cu") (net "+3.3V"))
 (segment (start 35.5092 29.0322) (end 35.5092 38.1) (width 0.0762) (layer "F.Cu") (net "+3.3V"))
 (segment (start 34.8996 29.0322) (end 34.8996 38.1) (width 0.0762) (layer "F.Cu") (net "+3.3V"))
 (segment (start 32.5374 38.1762) (end 32.6136 38.1) (width 0.0762) (layer "F.Cu") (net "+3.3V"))
 (segment (start 37.4904 29.0322) (end 37.5666 28.956) (width 0.0762) (layer "F.Cu") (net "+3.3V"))
 (segment (start 33.6804 38.1) (end 33.7566 38.1762) (width 0.0762) (layer "F.Cu") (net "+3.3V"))
 (segment (start 35.7378 28.956) (end 35.814 29.0322) (width 0.0762) (layer "F.Cu") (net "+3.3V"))
 (segment (start 34.2138 28.956) (end 34.29 29.0322) (width 0.0762) (layer "F.Cu") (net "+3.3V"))
 (segment (start 35.6616 29.0322) (end 35.7378 28.956) (width 0.0762) (layer "F.Cu") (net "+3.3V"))
 (segment (start 33.528 38.1) (end 33.528 29.0322) (width 0.0762) (layer "F.Cu") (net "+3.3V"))
 (segment (start 33.9852 38.1) (end 34.0614 38.1762) (width 0.0762) (layer "F.Cu") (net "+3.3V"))
 (segment (start 31.6992 38.1) (end 31.6992 29.0322) (width 0.0762) (layer "F.Cu") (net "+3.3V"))
 (segment (start 36.1188 38.1) (end 36.195 38.1762) (width 0.0762) (layer "F.Cu") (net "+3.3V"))
 (segment (start 35.9664 29.0322) (end 36.0426 28.956) (width 0.0762) (layer "F.Cu") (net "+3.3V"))
 (segment (start 34.1376 38.1) (end 34.1376 29.0322) (width 0.0762) (layer "F.Cu") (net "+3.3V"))
 (segment (start 38.5572 29.0322) (end 38.5572 39.1668) (width 0.0762) (layer "F.Cu") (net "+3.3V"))
 (segment (start 35.3568 38.1) (end 35.3568 29.0322) (width 0.0762) (layer "F.Cu") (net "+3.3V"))
 (segment (start 32.6136 38.1) (end 32.6136 29.0322) (width 0.0762) (layer "F.Cu") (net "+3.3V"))
 (segment (start 33.0708 38.1) (end 33.147 38.1762) (width 0.0762) (layer "F.Cu") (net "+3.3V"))
 (segment (start 32.1564 29.0322) (end 32.1564 38.1) (width 0.0762) (layer "F.Cu") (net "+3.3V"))
 (segment (start 31.9278 38.1762) (end 32.004 38.1) (width 0.0762) (layer "F.Cu") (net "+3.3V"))
 (segment (start 33.8328 38.1) (end 33.8328 29.0322) (width 0.0762) (layer "F.Cu") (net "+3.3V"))
 (segment (start 33.3756 29.0322) (end 33.3756 38.1) (width 0.0762) (layer "F.Cu") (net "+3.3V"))
 (segment (start 31.5468 38.1) (end 31.623 38.1762) (width 0.0762) (layer "F.Cu") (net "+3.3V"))
 (segment (start 37.1856 29.0322) (end 37.2618 28.956) (width 0.0762) (layer "F.Cu") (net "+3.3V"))
 (segment (start 38.0238 38.1762) (end 38.1 38.1) (width 0.0762) (layer "F.Cu") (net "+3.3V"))
 (segment (start 36.4998 38.1762) (end 36.576 38.1) (width 0.0762) (layer "F.Cu") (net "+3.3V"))
 (segment (start 35.3568 29.0322) (end 35.433 28.956) (width 0.0762) (layer "F.Cu") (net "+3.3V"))
 (segment (start 37.0332 29.0322) (end 37.0332 38.1) (width 0.0762) (layer "F.Cu") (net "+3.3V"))
 (segment (start 31.4706 28.956) (end 31.5468 29.0322) (width 0.0762) (layer "F.Cu") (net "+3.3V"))
 (segment (start 32.4612 29.0322) (end 32.4612 38.1) (width 0.0762) (layer "F.Cu") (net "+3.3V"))
 (segment (start 37.719 38.1762) (end 37.7952 38.1) (width 0.0762) (layer "F.Cu") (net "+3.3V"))
 (segment (start 34.8234 28.956) (end 34.8996 29.0322) (width 0.0762) (layer "F.Cu") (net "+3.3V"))
 (segment (start 33.6804 29.0322) (end 33.6804 38.1) (width 0.0762) (layer "F.Cu") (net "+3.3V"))
 (segment (start 33.147 38.1762) (end 33.2232 38.1) (width 0.0762) (layer "F.Cu") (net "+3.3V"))
 (segment (start 33.528 29.0322) (end 33.6042 28.956) (width 0.0762) (layer "F.Cu") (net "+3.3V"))
 (segment (start 35.2806 38.1762) (end 35.3568 38.1) (width 0.0762) (layer "F.Cu") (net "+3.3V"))
 (segment (start 37.1856 38.1) (end 37.1856 29.0322) (width 0.0762) (layer "F.Cu") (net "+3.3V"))
 (segment (start 34.1376 29.0322) (end 34.2138 28.956) (width 0.0762) (layer "F.Cu") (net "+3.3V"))
 (segment (start 35.2044 38.1) (end 35.2806 38.1762) (width 0.0762) (layer "F.Cu") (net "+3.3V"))
 (segment (start 34.29 38.1) (end 34.3662 38.1762) (width 0.0762) (layer "F.Cu") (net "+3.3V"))
 (segment (start 35.6616 38.1) (end 35.6616 29.0322) (width 0.0762) (layer "F.Cu") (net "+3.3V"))
 (segment (start 32.1564 38.1) (end 32.2326 38.1762) (width 0.0762) (layer "F.Cu") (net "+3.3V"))
 (segment (start 32.3088 38.1) (end 32.3088 29.0322) (width 0.0762) (layer "F.Cu") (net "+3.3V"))
 (segment (start 32.8422 38.1762) (end 32.9184 38.1) (width 0.0762) (layer "F.Cu") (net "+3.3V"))
 (segment (start 38.4048 29.0322) (end 38.481 28.956) (width 0.0762) (layer "F.Cu") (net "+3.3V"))
 (segment (start 38.2524 29.0322) (end 38.2524 38.1) (width 0.0762) (layer "F.Cu") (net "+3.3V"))
 (segment (start 32.2326 38.1762) (end 32.3088 38.1) (width 0.0762) (layer "F.Cu") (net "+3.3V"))
 (segment (start 30.7848 29.0322) (end 30.861 28.956) (width 0.0762) (layer "F.Cu") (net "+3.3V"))
 (segment (start 35.2044 29.0322) (end 35.2044 38.1) (width 0.0762) (layer "F.Cu") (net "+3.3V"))
 (segment (start 30.861 28.956) (end 30.9372 29.0322) (width 0.0762) (layer "F.Cu") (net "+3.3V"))
 (segment (start 32.4612 38.1) (end 32.5374 38.1762) (width 0.0762) (layer "F.Cu") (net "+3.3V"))
 (segment (start 37.7952 29.0322) (end 37.8714 28.956) (width 0.0762) (layer "F.Cu") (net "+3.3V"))
 (segment (start 32.0802 28.956) (end 32.1564 29.0322) (width 0.0762) (layer "F.Cu") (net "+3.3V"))
 (segment (start 36.8808 29.0322) (end 36.957 28.956) (width 0.0762) (layer "F.Cu") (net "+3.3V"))
 (segment (start 33.9852 29.0322) (end 33.9852 38.1) (width 0.0762) (layer "F.Cu") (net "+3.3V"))
 (segment (start 37.9476 29.0322) (end 37.9476 38.1) (width 0.0762) (layer "F.Cu") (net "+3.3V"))
 (segment (start 33.7566 38.1762) (end 33.8328 38.1) (width 0.0762) (layer "F.Cu") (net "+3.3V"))
 (segment (start 31.3182 38.1762) (end 31.3944 38.1) (width 0.0762) (layer "F.Cu") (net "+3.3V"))
 (segment (start 34.4424 29.0322) (end 34.5186 28.956) (width 0.0762) (layer "F.Cu") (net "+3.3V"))
 (segment (start 35.1282 28.956) (end 35.2044 29.0322) (width 0.0762) (layer "F.Cu") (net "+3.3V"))
 (segment (start 37.6428 38.1) (end 37.719 38.1762) (width 0.0762) (layer "F.Cu") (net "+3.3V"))
 (segment (start 37.338 29.0322) (end 37.338 38.1) (width 0.0762) (layer "F.Cu") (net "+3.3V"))
 (segment (start 37.5666 28.956) (end 37.6428 29.0322) (width 0.0762) (layer "F.Cu") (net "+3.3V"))
 (segment (start 36.2712 38.1) (end 36.2712 29.0322) (width 0.0762) (layer "F.Cu") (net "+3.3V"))
 (segment (start 34.29 29.0322) (end 34.29 38.1) (width 0.0762) (layer "F.Cu") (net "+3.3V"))
 (segment (start 36.195 38.1762) (end 36.2712 38.1) (width 0.0762) (layer "F.Cu") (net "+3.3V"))
 (segment (start 36.0426 28.956) (end 36.1188 29.0322) (width 0.0762) (layer "F.Cu") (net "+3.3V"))
 (segment (start 37.8714 28.956) (end 37.9476 29.0322) (width 0.0762) (layer "F.Cu") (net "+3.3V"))
 (segment (start 34.0614 38.1762) (end 34.1376 38.1) (width 0.0762) (layer "F.Cu") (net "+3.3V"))
 (segment (start 35.814 38.1) (end 35.8902 38.1762) (width 0.0762) (layer "F.Cu") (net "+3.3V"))
 (segment (start 34.3662 38.1762) (end 34.4424 38.1) (width 0.0762) (layer "F.Cu") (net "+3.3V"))
 (segment (start 32.3088 29.0322) (end 32.385 28.956) (width 0.0762) (layer "F.Cu") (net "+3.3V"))
 (segment (start 31.623 38.1762) (end 31.6992 38.1) (width 0.0762) (layer "F.Cu") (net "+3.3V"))
 (segment (start 30.9372 38.1) (end 31.0134 38.1762) (width 0.0762) (layer "F.Cu") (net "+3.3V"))
 (segment (start 32.9184 29.0322) (end 32.9946 28.956) (width 0.0762) (layer "F.Cu") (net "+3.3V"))
 (segment (start 37.4904 38.1) (end 37.4904 29.0322) (width 0.0762) (layer "F.Cu") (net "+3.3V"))
 (segment (start 34.5948 29.0322) (end 34.5948 38.1) (width 0.0762) (layer "F.Cu") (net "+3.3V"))
 (segment (start 35.052 29.0322) (end 35.1282 28.956) (width 0.0762) (layer "F.Cu") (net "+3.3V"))
 (segment (start 37.4142 38.1762) (end 37.4904 38.1) (width 0.0762) (layer "F.Cu") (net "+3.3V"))
 (segment (start 35.814 29.0322) (end 35.814 38.1) (width 0.0762) (layer "F.Cu") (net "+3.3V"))
 (segment (start 32.385 28.956) (end 32.4612 29.0322) (width 0.0762) (layer "F.Cu") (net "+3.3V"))
 (segment (start 37.7952 38.1) (end 37.7952 29.0322) (width 0.0762) (layer "F.Cu") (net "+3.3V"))
 (segment (start 36.3474 28.956) (end 36.4236 29.0322) (width 0.0762) (layer "F.Cu") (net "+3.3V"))
 (segment (start 32.766 38.1) (end 32.8422 38.1762) (width 0.0762) (layer "F.Cu") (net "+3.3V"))
 (segment (start 31.6992 29.0322) (end 31.7754 28.956) (width 0.0762) (layer "F.Cu") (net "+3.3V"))
 (segment (start 33.6042 28.956) (end 33.6804 29.0322) (width 0.0762) (layer "F.Cu") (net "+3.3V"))
 (segment (start 31.1658 28.956) (end 31.242 29.0322) (width 0.0762) (layer "F.Cu") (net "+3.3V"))
 (segment (start 31.5468 29.0322) (end 31.5468 38.1) (width 0.0762) (layer "F.Cu") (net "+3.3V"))
 (segment (start 32.9946 28.956) (end 33.0708 29.0322) (width 0.0762) (layer "F.Cu") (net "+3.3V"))
 (segment (start 34.5186 28.956) (end 34.5948 29.0322) (width 0.0762) (layer "F.Cu") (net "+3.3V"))
 (segment (start 37.0332 38.1) (end 37.1094 38.1762) (width 0.0762) (layer "F.Cu") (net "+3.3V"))
 (segment (start 31.242 38.1) (end 31.3182 38.1762) (width 0.0762) (layer "F.Cu") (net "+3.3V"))
 (segment (start 36.2712 29.0322) (end 36.3474 28.956) (width 0.0762) (layer "F.Cu") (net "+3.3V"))
 (segment (start 34.8996 38.1) (end 34.9758 38.1762) (width 0.0762) (layer "F.Cu") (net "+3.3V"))
 (segment (start 30.9372 29.0322) (end 30.9372 38.1) (width 0.0762) (layer "F.Cu") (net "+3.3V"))
 (segment (start 36.4236 29.0322) (end 36.4236 38.1) (width 0.0762) (layer "F.Cu") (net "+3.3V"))
 (segment (start 33.2994 28.956) (end 33.3756 29.0322) (width 0.0762) (layer "F.Cu") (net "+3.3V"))
 (segment (start 31.242 29.0322) (end 31.242 38.1) (width 0.0762) (layer "F.Cu") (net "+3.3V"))
 (segment (start 36.4236 38.1) (end 36.4998 38.1762) (width 0.0762) (layer "F.Cu") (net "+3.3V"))
 (segment (start 36.1188 29.0322) (end 36.1188 38.1) (width 0.0762) (layer "F.Cu") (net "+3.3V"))
 (segment (start 38.3286 38.1762) (end 38.4048 38.1) (width 0.0762) (layer "F.Cu") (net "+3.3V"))
 (segment (start 37.6428 29.0322) (end 37.6428 38.1) (width 0.0762) (layer "F.Cu") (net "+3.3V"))
 (segment (start 35.433 28.956) (end 35.5092 29.0322) (width 0.0762) (layer "F.Cu") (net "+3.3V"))
 (segment (start 36.8808 38.1) (end 36.8808 29.0322) (width 0.0762) (layer "F.Cu") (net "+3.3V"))
 (segment (start 35.9664 38.1) (end 35.9664 29.0322) (width 0.0762) (layer "F.Cu") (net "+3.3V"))
 (segment (start 34.7472 38.1) (end 34.7472 29.0322) (width 0.0762) (layer "F.Cu") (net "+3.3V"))
 (segment (start 31.3944 29.0322) (end 31.4706 28.956) (width 0.0762) (layer "F.Cu") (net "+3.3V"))
 (segment (start 36.576 38.1) (end 36.576 29.0322) (width 0.0762) (layer "F.Cu") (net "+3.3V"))
 (segment (start 32.6136 29.0322) (end 32.6898 28.956) (width 0.0762) (layer "F.Cu") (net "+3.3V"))
 (segment (start 38.1762 28.956) (end 38.2524 29.0322) (width 0.0762) (layer "F.Cu") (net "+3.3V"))
 (segment (start 33.2232 29.0322) (end 33.2994 28.956) (width 0.0762) (layer "F.Cu") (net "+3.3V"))
 (segment (start 38.1 38.1) (end 38.1 29.0322) (width 0.0762) (layer "F.Cu") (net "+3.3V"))
 (segment (start 31.8516 29.0322) (end 31.8516 38.1) (width 0.0762) (layer "F.Cu") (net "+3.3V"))
 (segment (start 36.7284 38.1) (end 36.8046 38.1762) (width 0.0762) (layer "F.Cu") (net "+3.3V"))
 (segment (start 34.9758 38.1762) (end 35.052 38.1) (width 0.0762) (layer "F.Cu") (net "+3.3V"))
 (segment (start 37.1094 38.1762) (end 37.1856 38.1) (width 0.0762) (layer "F.Cu") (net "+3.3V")))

